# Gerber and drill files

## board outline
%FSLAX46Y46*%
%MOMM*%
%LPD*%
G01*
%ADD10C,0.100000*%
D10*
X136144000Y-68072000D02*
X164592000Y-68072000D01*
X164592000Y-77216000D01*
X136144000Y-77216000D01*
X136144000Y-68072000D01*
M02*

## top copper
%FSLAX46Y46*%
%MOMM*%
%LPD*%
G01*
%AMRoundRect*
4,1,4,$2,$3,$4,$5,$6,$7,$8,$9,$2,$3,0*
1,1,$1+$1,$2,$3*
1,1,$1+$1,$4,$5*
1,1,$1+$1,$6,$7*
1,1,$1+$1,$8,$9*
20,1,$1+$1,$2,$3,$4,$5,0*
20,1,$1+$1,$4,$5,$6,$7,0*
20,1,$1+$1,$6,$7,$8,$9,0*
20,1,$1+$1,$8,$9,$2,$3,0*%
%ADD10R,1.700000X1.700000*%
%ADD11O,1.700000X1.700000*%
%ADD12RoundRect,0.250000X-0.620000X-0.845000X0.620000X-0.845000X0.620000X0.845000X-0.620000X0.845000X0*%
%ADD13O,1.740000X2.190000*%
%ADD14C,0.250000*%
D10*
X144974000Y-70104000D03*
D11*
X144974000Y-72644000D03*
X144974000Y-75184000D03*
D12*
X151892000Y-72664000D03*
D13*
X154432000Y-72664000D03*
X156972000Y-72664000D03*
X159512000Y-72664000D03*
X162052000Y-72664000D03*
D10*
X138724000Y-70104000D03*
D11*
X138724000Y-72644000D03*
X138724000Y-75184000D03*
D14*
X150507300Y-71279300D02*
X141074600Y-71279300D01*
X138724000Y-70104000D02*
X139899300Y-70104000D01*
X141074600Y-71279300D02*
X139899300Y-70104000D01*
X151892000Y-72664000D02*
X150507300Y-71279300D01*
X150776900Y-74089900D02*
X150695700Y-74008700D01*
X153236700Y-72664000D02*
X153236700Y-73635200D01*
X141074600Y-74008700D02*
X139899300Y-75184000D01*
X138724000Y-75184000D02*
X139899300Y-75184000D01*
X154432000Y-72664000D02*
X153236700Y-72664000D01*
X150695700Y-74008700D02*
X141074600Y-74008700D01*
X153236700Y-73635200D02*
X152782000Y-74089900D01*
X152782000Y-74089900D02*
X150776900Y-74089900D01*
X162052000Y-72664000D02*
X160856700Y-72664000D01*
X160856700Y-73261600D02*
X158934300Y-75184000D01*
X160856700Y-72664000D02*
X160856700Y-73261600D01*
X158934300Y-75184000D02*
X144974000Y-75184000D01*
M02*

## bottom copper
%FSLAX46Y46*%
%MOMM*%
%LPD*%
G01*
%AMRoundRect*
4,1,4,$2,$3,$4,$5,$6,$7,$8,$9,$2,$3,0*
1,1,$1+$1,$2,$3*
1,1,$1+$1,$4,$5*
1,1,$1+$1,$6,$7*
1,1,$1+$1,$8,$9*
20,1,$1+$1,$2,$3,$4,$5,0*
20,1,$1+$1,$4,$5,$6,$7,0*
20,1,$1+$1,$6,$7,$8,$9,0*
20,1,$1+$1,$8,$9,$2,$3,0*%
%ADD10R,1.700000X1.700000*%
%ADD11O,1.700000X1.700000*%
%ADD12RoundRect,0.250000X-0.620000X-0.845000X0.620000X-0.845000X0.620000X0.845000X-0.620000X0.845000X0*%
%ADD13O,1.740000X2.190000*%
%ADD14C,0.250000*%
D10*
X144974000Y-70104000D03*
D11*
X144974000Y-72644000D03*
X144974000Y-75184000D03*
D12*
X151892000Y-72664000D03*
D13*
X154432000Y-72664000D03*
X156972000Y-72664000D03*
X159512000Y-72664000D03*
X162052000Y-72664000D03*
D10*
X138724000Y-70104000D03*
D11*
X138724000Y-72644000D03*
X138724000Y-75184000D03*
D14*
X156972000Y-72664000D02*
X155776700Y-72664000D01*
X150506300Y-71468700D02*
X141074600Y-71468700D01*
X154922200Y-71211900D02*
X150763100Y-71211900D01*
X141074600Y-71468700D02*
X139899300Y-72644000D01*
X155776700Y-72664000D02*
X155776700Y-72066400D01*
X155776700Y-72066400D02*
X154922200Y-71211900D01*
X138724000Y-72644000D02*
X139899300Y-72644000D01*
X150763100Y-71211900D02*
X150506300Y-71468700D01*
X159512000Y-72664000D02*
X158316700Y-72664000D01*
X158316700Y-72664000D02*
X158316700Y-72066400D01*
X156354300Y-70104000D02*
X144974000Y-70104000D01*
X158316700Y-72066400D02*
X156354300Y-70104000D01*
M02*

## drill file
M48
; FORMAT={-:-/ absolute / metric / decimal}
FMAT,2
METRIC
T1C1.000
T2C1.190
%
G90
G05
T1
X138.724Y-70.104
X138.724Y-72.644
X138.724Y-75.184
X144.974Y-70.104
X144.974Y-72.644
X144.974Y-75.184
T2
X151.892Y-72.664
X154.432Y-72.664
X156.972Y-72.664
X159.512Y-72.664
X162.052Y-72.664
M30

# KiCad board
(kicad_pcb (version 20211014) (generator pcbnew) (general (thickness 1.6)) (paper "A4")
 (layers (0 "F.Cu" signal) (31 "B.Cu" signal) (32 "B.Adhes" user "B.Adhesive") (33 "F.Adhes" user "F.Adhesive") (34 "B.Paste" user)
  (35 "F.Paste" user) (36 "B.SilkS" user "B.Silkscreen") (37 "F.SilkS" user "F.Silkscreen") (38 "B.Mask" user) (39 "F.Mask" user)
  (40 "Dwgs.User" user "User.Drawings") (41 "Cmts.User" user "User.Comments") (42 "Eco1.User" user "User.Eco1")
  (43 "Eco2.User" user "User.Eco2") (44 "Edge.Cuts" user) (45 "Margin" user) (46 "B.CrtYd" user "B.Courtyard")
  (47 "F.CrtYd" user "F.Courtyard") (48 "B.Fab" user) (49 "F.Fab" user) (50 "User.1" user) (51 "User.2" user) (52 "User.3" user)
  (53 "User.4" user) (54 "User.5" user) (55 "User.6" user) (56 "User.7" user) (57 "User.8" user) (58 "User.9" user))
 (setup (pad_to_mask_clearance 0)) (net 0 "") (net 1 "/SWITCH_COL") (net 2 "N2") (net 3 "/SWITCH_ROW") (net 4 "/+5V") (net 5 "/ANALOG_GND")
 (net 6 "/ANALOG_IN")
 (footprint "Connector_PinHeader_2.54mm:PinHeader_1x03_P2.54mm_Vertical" (layer "F.Cu") (at 144.974 70.104)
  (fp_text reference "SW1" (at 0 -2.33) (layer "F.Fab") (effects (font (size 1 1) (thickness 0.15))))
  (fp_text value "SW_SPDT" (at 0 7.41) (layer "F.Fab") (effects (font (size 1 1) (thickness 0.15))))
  (pad "1" thru_hole rect (at 0 0) (size 1.7 1.7) (drill 1) (layers *.Cu *.Mask) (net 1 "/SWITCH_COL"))
  (pad "2" thru_hole oval (at 0 2.54) (size 1.7 1.7) (drill 1) (layers *.Cu *.Mask) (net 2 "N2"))
  (pad "3" thru_hole oval (at 0 5.08) (size 1.7 1.7) (drill 1) (layers *.Cu *.Mask) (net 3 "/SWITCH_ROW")))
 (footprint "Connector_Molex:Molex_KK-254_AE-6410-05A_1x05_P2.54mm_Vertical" (layer "F.Cu") (at 151.892 72.664)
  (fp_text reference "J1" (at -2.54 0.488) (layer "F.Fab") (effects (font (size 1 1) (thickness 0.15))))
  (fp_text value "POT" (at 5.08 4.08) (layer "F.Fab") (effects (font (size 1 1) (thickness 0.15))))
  (pad "1" thru_hole roundrect (at 0 0) (size 1.74 2.19) (drill 1.19) (layers *.Cu *.Mask) (roundrect_rratio 0.1436781609) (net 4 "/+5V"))
  (pad "2" thru_hole oval (at 2.54 0) (size 1.74 2.19) (drill 1.19) (layers *.Cu *.Mask) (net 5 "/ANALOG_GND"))
  (pad "3" thru_hole oval (at 5.08 0) (size 1.74 2.19) (drill 1.19) (layers *.Cu *.Mask) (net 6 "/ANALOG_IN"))
  (pad "4" thru_hole oval (at 7.62 0) (size 1.74 2.19) (drill 1.19) (layers *.Cu *.Mask) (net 1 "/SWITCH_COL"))
  (pad "5" thru_hole oval (at 10.16 0) (size 1.74 2.19) (drill 1.19) (layers *.Cu *.Mask) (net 3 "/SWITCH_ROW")))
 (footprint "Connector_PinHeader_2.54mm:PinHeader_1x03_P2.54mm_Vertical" (layer "F.Cu") (at 138.724 70.104)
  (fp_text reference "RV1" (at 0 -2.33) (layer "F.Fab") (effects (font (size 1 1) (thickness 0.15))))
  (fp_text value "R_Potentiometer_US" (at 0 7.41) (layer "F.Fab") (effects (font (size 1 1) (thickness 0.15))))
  (pad "1" thru_hole rect (at 0 0) (size 1.7 1.7) (drill 1) (layers *.Cu *.Mask) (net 4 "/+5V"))
  (pad "2" thru_hole oval (at 0 2.54) (size 1.7 1.7) (drill 1) (layers *.Cu *.Mask) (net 6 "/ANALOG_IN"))
  (pad "3" thru_hole oval (at 0 5.08) (size 1.7 1.7) (drill 1) (layers *.Cu *.Mask) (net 5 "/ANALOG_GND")))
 (gr_rect (start 136.144 68.072) (end 164.592 77.216) (layer "Edge.Cuts") (width 0.1) (fill none))
 (segment (start 150.5073 71.2793) (end 141.0746 71.2793) (width 0.25) (layer "F.Cu") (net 4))
 (segment (start 138.724 70.104) (end 139.8993 70.104) (width 0.25) (layer "F.Cu") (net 4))
 (segment (start 141.0746 71.2793) (end 139.8993 70.104) (width 0.25) (layer "F.Cu") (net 4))
 (segment (start 151.892 72.664) (end 150.5073 71.2793) (width 0.25) (layer "F.Cu") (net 4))
 (segment (start 150.7769 74.0899) (end 150.6957 74.0087) (width 0.25) (layer "F.Cu") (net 5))
 (segment (start 153.2367 72.664) (end 153.2367 73.6352) (width 0.25) (layer "F.Cu") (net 5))
 (segment (start 141.0746 74.0087) (end 139.8993 75.184) (width 0.25) (layer "F.Cu") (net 5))
 (segment (start 138.724 75.184) (end 139.8993 75.184) (width 0.25) (layer "F.Cu") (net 5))
 (segment (start 154.432 72.664) (end 153.2367 72.664) (width 0.25) (layer "F.Cu") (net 5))
 (segment (start 150.6957 74.0087) (end 141.0746 74.0087) (width 0.25) (layer "F.Cu") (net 5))
 (segment (start 153.2367 73.6352) (end 152.782 74.0899) (width 0.25) (layer "F.Cu") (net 5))
 (segment (start 152.782 74.0899) (end 150.7769 74.0899) (width 0.25) (layer "F.Cu") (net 5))
 (segment (start 156.972 72.664) (end 155.7767 72.664) (width 0.25) (layer "B.Cu") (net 6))
 (segment (start 150.5063 71.4687) (end 141.0746 71.4687) (width 0.25) (layer "B.Cu") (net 6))
 (segment (start 154.9222 71.2119) (end 150.7631 71.2119) (width 0.25) (layer "B.Cu") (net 6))
 (segment (start 141.0746 71.4687) (end 139.8993 72.644) (width 0.25) (layer "B.Cu") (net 6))
 (segment (start 155.7767 72.664) (end 155.7767 72.0664) (width 0.25) (layer "B.Cu") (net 6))
 (segment (start 155.7767 72.0664) (end 154.9222 71.2119) (width 0.25) (layer "B.Cu") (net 6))
 (segment (start 138.724 72.644) (end 139.8993 72.644) (width 0.25) (layer "B.Cu") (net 6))
 (segment (start 150.7631 71.2119) (end 150.5063 71.4687) (width 0.25) (layer "B.Cu") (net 6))
 (segment (start 159.512 72.664) (end 158.3167 72.664) (width 0.25) (layer "B.Cu") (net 1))
 (segment (start 158.3167 72.664) (end 158.3167 72.0664) (width 0.25) (layer "B.Cu") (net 1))
 (segment (start 156.3543 70.104) (end 144.974 70.104) (width 0.25) (layer "B.Cu") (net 1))
 (segment (start 158.3167 72.0664) (end 156.3543 70.104) (width 0.25) (layer "B.Cu") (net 1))
 (segment (start 162.052 72.664) (end 160.8567 72.664) (width 0.25) (layer "F.Cu") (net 3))
 (segment (start 160.8567 73.2616) (end 158.9343 75.184) (width 0.25) (layer "F.Cu") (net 3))
 (segment (start 160.8567 72.664) (end 160.8567 73.2616) (width 0.25) (layer "F.Cu") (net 3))
 (segment (start 158.9343 75.184) (end 144.974 75.184) (width 0.25) (layer "F.Cu") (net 3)))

